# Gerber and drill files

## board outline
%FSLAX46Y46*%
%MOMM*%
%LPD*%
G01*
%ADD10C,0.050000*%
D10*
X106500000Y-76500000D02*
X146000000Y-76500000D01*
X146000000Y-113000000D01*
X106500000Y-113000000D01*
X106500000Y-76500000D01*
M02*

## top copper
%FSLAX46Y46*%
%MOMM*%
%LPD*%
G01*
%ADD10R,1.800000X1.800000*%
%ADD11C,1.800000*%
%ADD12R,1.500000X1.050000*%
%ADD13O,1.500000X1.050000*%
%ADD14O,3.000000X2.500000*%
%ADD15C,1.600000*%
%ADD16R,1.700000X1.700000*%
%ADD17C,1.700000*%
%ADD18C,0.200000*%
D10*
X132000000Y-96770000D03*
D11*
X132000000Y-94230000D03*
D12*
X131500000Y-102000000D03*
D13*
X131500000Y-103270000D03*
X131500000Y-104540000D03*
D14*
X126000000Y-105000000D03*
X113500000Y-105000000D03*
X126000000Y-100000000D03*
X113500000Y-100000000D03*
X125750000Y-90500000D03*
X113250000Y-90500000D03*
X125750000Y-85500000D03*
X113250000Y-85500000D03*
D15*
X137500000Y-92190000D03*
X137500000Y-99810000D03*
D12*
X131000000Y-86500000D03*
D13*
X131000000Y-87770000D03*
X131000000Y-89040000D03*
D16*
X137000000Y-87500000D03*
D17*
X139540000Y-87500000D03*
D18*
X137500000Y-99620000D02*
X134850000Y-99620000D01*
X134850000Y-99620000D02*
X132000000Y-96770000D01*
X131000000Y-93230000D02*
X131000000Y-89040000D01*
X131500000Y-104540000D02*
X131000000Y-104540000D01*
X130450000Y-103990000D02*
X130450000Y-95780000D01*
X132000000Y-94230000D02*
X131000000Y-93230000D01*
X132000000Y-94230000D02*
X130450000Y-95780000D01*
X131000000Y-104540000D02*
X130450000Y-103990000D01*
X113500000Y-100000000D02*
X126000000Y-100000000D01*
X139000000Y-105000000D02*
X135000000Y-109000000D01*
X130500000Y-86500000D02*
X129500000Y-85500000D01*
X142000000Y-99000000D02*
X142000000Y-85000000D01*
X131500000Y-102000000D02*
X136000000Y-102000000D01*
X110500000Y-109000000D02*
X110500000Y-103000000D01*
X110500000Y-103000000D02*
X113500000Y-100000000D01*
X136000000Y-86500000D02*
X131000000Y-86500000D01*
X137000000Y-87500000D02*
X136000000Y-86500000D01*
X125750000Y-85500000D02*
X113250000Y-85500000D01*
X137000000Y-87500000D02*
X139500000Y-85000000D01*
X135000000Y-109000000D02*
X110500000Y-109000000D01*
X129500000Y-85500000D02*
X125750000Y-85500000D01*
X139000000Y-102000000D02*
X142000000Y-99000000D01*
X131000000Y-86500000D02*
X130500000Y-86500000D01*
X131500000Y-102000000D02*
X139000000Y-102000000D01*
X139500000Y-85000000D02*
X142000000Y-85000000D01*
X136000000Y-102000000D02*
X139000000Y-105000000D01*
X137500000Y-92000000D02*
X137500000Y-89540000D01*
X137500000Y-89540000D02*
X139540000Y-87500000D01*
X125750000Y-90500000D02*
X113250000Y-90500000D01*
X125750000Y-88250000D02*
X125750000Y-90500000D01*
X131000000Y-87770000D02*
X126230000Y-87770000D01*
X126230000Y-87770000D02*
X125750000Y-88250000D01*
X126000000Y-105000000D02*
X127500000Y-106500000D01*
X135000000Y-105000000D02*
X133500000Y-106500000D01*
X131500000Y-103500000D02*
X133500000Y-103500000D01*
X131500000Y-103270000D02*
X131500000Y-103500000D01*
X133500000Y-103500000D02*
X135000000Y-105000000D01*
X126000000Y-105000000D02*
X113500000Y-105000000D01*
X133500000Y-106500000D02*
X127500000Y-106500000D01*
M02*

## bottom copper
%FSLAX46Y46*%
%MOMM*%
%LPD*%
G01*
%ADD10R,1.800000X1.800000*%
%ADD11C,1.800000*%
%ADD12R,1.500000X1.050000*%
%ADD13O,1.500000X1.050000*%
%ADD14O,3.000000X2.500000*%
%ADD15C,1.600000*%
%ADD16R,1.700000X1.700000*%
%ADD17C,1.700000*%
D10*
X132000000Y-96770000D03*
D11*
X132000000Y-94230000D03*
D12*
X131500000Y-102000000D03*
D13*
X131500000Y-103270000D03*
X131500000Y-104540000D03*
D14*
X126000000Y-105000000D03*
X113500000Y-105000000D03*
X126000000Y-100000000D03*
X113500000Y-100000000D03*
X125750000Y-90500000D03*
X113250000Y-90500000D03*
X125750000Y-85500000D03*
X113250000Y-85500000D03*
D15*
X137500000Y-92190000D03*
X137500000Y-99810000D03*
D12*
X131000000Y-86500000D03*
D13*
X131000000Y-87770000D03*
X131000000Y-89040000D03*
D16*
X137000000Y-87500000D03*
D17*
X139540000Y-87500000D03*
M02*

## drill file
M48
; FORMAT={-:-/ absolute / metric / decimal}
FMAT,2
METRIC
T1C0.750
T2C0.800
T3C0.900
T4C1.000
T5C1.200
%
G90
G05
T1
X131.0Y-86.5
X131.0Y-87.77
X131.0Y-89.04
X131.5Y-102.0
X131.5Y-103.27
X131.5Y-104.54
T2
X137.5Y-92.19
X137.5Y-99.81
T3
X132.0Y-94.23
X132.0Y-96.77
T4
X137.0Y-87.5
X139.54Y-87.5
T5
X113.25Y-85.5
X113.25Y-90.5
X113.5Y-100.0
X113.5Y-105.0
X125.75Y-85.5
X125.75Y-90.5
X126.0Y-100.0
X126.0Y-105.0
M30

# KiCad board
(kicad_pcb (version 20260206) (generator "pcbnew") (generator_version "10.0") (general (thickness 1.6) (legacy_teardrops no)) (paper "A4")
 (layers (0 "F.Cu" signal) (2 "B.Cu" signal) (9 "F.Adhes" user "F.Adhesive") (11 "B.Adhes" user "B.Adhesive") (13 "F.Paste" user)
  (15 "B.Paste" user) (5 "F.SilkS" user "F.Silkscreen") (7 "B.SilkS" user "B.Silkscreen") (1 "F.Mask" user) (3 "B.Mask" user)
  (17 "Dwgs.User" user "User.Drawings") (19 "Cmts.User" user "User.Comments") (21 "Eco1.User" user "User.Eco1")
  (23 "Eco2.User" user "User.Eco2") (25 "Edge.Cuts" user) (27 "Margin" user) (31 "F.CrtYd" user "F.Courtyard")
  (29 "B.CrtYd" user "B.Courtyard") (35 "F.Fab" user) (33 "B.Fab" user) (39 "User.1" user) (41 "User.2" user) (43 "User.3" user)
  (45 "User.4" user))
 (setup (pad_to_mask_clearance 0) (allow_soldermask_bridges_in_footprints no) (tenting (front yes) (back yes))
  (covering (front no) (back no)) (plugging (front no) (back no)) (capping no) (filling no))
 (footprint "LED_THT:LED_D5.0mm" (layer "F.Cu") (at 132 96.77 90)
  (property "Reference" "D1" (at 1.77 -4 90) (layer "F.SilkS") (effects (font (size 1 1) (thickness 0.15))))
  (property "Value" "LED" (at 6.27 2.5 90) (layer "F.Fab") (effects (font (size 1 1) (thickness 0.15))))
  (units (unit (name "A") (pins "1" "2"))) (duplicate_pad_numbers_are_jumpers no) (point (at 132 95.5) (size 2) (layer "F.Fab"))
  (pad "1" thru_hole rect (at 0 0 90) (size 1.8 1.8) (drill 0.9) (layers "*.Cu" "*.Mask") (remove_unused_layers no) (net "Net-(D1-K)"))
  (pad "2" thru_hole circle (at 2.54 0 90) (size 1.8 1.8) (drill 0.9) (layers "*.Cu" "*.Mask") (remove_unused_layers no) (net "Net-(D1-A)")))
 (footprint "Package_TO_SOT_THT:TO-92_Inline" (layer "F.Cu") (at 131.5 102 -90)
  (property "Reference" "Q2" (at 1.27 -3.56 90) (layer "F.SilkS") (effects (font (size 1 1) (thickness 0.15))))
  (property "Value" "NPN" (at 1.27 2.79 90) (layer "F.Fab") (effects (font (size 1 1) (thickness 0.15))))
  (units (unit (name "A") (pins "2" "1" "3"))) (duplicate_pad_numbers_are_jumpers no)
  (pad "1" thru_hole rect (at 0 0 270) (size 1.05 1.5) (drill 0.75) (layers "*.Cu" "*.Mask") (remove_unused_layers no) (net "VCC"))
  (pad "2" thru_hole oval (at 1.27 0 270) (size 1.05 1.5) (drill 0.75) (layers "*.Cu" "*.Mask") (remove_unused_layers no) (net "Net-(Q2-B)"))
  (pad "3" thru_hole oval (at 2.54 0 270) (size 1.05 1.5) (drill 0.75) (layers "*.Cu" "*.Mask") (remove_unused_layers no) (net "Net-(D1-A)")))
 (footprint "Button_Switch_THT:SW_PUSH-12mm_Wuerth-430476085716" (layer "F.Cu") (at 126 105 180)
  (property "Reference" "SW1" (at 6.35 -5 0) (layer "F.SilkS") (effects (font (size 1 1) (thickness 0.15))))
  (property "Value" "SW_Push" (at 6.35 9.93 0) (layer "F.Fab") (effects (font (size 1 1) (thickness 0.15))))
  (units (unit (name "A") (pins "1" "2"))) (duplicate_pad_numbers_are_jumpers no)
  (pad "1" thru_hole oval (at 0 0 180) (size 3 2.5) (drill 1.2) (layers "*.Cu" "*.Mask") (remove_unused_layers no) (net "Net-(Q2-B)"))
  (pad "1" thru_hole oval (at 12.5 0 180) (size 3 2.5) (drill 1.2) (layers "*.Cu" "*.Mask") (remove_unused_layers no) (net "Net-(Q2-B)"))
  (pad "2" thru_hole oval (at 0 5 180) (size 3 2.5) (drill 1.2) (layers "*.Cu" "*.Mask") (remove_unused_layers no) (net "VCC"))
  (pad "2" thru_hole oval (at 12.5 5 180) (size 3 2.5) (drill 1.2) (layers "*.Cu" "*.Mask") (remove_unused_layers no) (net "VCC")))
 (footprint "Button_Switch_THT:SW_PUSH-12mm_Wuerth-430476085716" (layer "F.Cu") (at 125.75 90.5 180)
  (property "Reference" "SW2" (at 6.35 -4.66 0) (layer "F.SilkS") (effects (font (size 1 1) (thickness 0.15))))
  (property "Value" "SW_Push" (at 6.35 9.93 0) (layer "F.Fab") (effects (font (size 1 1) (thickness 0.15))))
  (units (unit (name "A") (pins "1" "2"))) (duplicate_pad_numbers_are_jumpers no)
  (pad "1" thru_hole oval (at 0 0 180) (size 3 2.5) (drill 1.2) (layers "*.Cu" "*.Mask") (remove_unused_layers no) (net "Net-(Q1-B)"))
  (pad "1" thru_hole oval (at 12.5 0 180) (size 3 2.5) (drill 1.2) (layers "*.Cu" "*.Mask") (remove_unused_layers no) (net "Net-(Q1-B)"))
  (pad "2" thru_hole oval (at 0 5 180) (size 3 2.5) (drill 1.2) (layers "*.Cu" "*.Mask") (remove_unused_layers no) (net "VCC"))
  (pad "2" thru_hole oval (at 12.5 5 180) (size 3 2.5) (drill 1.2) (layers "*.Cu" "*.Mask") (remove_unused_layers no) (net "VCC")))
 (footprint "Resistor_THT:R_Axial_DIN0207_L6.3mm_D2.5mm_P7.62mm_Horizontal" (layer "F.Cu") (at 137.5 92.19 -90)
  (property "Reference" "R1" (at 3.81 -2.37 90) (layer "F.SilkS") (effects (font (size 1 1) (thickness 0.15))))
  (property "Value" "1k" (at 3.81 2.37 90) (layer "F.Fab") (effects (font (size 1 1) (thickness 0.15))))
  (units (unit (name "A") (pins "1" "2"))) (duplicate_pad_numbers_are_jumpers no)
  (pad "1" thru_hole circle (at 0 0 270) (size 1.6 1.6) (drill 0.8) (layers "*.Cu" "*.Mask") (remove_unused_layers no) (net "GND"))
  (pad "2" thru_hole circle (at 7.62 0 270) (size 1.6 1.6) (drill 0.8) (layers "*.Cu" "*.Mask") (remove_unused_layers no) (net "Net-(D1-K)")))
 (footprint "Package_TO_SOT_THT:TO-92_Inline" (layer "F.Cu") (at 131 86.5 -90)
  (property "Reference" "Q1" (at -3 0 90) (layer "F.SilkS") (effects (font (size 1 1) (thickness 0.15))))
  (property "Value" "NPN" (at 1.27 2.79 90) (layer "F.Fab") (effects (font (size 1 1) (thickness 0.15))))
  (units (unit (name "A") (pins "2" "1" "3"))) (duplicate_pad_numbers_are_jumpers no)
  (pad "1" thru_hole rect (at 0 0 270) (size 1.05 1.5) (drill 0.75) (layers "*.Cu" "*.Mask") (remove_unused_layers no) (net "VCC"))
  (pad "2" thru_hole oval (at 1.27 0 270) (size 1.05 1.5) (drill 0.75) (layers "*.Cu" "*.Mask") (remove_unused_layers no) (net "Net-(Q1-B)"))
  (pad "3" thru_hole oval (at 2.54 0 270) (size 1.05 1.5) (drill 0.75) (layers "*.Cu" "*.Mask") (remove_unused_layers no) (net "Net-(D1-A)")))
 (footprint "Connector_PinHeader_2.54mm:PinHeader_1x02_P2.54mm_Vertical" (layer "F.Cu") (at 137 87.5 90)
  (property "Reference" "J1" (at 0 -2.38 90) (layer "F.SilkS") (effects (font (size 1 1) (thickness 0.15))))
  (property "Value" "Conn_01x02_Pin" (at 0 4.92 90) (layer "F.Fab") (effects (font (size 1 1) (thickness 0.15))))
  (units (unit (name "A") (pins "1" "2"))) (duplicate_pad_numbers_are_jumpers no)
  (pad "1" thru_hole rect (at 0 0 90) (size 1.7 1.7) (drill 1) (layers "*.Cu" "*.Mask") (remove_unused_layers no) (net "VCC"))
  (pad "2" thru_hole circle (at 0 2.54 90) (size 1.7 1.7) (drill 1) (layers "*.Cu" "*.Mask") (remove_unused_layers no) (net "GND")))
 (gr_rect (start 106.5 76.5) (end 146 113) (stroke (width 0.05) (type default)) (fill no) (layer "Edge.Cuts"))
 (segment (start 137.5 99.62) (end 134.85 99.62) (width 0.2) (layer "F.Cu") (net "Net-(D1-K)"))
 (segment (start 134.85 99.62) (end 132 96.77) (width 0.2) (layer "F.Cu") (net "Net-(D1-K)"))
 (segment (start 131 93.23) (end 131 89.04) (width 0.2) (layer "F.Cu") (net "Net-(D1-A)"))
 (segment (start 131.5 104.54) (end 131 104.54) (width 0.2) (layer "F.Cu") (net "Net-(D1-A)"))
 (segment (start 130.45 103.99) (end 130.45 95.78) (width 0.2) (layer "F.Cu") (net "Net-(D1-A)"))
 (segment (start 132 94.23) (end 131 93.23) (width 0.2) (layer "F.Cu") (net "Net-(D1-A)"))
 (segment (start 132 94.23) (end 130.45 95.78) (width 0.2) (layer "F.Cu") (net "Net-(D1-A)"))
 (segment (start 131 104.54) (end 130.45 103.99) (width 0.2) (layer "F.Cu") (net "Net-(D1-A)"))
 (segment (start 113.5 100) (end 126 100) (width 0.2) (layer "F.Cu") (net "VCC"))
 (segment (start 139 105) (end 135 109) (width 0.2) (layer "F.Cu") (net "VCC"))
 (segment (start 130.5 86.5) (end 129.5 85.5) (width 0.2) (layer "F.Cu") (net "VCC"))
 (segment (start 142 99) (end 142 85) (width 0.2) (layer "F.Cu") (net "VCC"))
 (segment (start 131.5 102) (end 136 102) (width 0.2) (layer "F.Cu") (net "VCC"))
 (segment (start 110.5 109) (end 110.5 103) (width 0.2) (layer "F.Cu") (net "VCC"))
 (segment (start 110.5 103) (end 113.5 100) (width 0.2) (layer "F.Cu") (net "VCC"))
 (segment (start 136 86.5) (end 131 86.5) (width 0.2) (layer "F.Cu") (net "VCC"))
 (segment (start 137 87.5) (end 136 86.5) (width 0.2) (layer "F.Cu") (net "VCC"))
 (segment (start 125.75 85.5) (end 113.25 85.5) (width 0.2) (layer "F.Cu") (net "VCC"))
 (segment (start 137 87.5) (end 139.5 85) (width 0.2) (layer "F.Cu") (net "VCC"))
 (segment (start 135 109) (end 110.5 109) (width 0.2) (layer "F.Cu") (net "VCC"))
 (segment (start 129.5 85.5) (end 125.75 85.5) (width 0.2) (layer "F.Cu") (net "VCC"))
 (segment (start 139 102) (end 142 99) (width 0.2) (layer "F.Cu") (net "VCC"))
 (segment (start 131 86.5) (end 130.5 86.5) (width 0.2) (layer "F.Cu") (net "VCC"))
 (segment (start 131.5 102) (end 139 102) (width 0.2) (layer "F.Cu") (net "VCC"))
 (segment (start 139.5 85) (end 142 85) (width 0.2) (layer "F.Cu") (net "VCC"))
 (segment (start 136 102) (end 139 105) (width 0.2) (layer "F.Cu") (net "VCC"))
 (segment (start 137.5 92) (end 137.5 89.54) (width 0.2) (layer "F.Cu") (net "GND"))
 (segment (start 137.5 89.54) (end 139.54 87.5) (width 0.2) (layer "F.Cu") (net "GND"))
 (segment (start 125.75 90.5) (end 113.25 90.5) (width 0.2) (layer "F.Cu") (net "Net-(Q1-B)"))
 (segment (start 125.75 88.25) (end 125.75 90.5) (width 0.2) (layer "F.Cu") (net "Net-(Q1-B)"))
 (segment (start 131 87.77) (end 126.23 87.77) (width 0.2) (layer "F.Cu") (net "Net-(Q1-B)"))
 (segment (start 126.23 87.77) (end 125.75 88.25) (width 0.2) (layer "F.Cu") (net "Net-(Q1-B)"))
 (segment (start 126 105) (end 127.5 106.5) (width 0.2) (layer "F.Cu") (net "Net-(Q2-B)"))
 (segment (start 135 105) (end 133.5 106.5) (width 0.2) (layer "F.Cu") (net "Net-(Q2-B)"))
 (segment (start 131.5 103.5) (end 133.5 103.5) (width 0.2) (layer "F.Cu") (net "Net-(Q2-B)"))
 (segment (start 131.5 103.27) (end 131.5 103.5) (width 0.2) (layer "F.Cu") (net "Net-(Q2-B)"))
 (segment (start 133.5 103.5) (end 135 105) (width 0.2) (layer "F.Cu") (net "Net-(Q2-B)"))
 (segment (start 126 105) (end 113.5 105) (width 0.2) (layer "F.Cu") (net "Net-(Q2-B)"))
 (segment (start 133.5 106.5) (end 127.5 106.5) (width 0.2) (layer "F.Cu") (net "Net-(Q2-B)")))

